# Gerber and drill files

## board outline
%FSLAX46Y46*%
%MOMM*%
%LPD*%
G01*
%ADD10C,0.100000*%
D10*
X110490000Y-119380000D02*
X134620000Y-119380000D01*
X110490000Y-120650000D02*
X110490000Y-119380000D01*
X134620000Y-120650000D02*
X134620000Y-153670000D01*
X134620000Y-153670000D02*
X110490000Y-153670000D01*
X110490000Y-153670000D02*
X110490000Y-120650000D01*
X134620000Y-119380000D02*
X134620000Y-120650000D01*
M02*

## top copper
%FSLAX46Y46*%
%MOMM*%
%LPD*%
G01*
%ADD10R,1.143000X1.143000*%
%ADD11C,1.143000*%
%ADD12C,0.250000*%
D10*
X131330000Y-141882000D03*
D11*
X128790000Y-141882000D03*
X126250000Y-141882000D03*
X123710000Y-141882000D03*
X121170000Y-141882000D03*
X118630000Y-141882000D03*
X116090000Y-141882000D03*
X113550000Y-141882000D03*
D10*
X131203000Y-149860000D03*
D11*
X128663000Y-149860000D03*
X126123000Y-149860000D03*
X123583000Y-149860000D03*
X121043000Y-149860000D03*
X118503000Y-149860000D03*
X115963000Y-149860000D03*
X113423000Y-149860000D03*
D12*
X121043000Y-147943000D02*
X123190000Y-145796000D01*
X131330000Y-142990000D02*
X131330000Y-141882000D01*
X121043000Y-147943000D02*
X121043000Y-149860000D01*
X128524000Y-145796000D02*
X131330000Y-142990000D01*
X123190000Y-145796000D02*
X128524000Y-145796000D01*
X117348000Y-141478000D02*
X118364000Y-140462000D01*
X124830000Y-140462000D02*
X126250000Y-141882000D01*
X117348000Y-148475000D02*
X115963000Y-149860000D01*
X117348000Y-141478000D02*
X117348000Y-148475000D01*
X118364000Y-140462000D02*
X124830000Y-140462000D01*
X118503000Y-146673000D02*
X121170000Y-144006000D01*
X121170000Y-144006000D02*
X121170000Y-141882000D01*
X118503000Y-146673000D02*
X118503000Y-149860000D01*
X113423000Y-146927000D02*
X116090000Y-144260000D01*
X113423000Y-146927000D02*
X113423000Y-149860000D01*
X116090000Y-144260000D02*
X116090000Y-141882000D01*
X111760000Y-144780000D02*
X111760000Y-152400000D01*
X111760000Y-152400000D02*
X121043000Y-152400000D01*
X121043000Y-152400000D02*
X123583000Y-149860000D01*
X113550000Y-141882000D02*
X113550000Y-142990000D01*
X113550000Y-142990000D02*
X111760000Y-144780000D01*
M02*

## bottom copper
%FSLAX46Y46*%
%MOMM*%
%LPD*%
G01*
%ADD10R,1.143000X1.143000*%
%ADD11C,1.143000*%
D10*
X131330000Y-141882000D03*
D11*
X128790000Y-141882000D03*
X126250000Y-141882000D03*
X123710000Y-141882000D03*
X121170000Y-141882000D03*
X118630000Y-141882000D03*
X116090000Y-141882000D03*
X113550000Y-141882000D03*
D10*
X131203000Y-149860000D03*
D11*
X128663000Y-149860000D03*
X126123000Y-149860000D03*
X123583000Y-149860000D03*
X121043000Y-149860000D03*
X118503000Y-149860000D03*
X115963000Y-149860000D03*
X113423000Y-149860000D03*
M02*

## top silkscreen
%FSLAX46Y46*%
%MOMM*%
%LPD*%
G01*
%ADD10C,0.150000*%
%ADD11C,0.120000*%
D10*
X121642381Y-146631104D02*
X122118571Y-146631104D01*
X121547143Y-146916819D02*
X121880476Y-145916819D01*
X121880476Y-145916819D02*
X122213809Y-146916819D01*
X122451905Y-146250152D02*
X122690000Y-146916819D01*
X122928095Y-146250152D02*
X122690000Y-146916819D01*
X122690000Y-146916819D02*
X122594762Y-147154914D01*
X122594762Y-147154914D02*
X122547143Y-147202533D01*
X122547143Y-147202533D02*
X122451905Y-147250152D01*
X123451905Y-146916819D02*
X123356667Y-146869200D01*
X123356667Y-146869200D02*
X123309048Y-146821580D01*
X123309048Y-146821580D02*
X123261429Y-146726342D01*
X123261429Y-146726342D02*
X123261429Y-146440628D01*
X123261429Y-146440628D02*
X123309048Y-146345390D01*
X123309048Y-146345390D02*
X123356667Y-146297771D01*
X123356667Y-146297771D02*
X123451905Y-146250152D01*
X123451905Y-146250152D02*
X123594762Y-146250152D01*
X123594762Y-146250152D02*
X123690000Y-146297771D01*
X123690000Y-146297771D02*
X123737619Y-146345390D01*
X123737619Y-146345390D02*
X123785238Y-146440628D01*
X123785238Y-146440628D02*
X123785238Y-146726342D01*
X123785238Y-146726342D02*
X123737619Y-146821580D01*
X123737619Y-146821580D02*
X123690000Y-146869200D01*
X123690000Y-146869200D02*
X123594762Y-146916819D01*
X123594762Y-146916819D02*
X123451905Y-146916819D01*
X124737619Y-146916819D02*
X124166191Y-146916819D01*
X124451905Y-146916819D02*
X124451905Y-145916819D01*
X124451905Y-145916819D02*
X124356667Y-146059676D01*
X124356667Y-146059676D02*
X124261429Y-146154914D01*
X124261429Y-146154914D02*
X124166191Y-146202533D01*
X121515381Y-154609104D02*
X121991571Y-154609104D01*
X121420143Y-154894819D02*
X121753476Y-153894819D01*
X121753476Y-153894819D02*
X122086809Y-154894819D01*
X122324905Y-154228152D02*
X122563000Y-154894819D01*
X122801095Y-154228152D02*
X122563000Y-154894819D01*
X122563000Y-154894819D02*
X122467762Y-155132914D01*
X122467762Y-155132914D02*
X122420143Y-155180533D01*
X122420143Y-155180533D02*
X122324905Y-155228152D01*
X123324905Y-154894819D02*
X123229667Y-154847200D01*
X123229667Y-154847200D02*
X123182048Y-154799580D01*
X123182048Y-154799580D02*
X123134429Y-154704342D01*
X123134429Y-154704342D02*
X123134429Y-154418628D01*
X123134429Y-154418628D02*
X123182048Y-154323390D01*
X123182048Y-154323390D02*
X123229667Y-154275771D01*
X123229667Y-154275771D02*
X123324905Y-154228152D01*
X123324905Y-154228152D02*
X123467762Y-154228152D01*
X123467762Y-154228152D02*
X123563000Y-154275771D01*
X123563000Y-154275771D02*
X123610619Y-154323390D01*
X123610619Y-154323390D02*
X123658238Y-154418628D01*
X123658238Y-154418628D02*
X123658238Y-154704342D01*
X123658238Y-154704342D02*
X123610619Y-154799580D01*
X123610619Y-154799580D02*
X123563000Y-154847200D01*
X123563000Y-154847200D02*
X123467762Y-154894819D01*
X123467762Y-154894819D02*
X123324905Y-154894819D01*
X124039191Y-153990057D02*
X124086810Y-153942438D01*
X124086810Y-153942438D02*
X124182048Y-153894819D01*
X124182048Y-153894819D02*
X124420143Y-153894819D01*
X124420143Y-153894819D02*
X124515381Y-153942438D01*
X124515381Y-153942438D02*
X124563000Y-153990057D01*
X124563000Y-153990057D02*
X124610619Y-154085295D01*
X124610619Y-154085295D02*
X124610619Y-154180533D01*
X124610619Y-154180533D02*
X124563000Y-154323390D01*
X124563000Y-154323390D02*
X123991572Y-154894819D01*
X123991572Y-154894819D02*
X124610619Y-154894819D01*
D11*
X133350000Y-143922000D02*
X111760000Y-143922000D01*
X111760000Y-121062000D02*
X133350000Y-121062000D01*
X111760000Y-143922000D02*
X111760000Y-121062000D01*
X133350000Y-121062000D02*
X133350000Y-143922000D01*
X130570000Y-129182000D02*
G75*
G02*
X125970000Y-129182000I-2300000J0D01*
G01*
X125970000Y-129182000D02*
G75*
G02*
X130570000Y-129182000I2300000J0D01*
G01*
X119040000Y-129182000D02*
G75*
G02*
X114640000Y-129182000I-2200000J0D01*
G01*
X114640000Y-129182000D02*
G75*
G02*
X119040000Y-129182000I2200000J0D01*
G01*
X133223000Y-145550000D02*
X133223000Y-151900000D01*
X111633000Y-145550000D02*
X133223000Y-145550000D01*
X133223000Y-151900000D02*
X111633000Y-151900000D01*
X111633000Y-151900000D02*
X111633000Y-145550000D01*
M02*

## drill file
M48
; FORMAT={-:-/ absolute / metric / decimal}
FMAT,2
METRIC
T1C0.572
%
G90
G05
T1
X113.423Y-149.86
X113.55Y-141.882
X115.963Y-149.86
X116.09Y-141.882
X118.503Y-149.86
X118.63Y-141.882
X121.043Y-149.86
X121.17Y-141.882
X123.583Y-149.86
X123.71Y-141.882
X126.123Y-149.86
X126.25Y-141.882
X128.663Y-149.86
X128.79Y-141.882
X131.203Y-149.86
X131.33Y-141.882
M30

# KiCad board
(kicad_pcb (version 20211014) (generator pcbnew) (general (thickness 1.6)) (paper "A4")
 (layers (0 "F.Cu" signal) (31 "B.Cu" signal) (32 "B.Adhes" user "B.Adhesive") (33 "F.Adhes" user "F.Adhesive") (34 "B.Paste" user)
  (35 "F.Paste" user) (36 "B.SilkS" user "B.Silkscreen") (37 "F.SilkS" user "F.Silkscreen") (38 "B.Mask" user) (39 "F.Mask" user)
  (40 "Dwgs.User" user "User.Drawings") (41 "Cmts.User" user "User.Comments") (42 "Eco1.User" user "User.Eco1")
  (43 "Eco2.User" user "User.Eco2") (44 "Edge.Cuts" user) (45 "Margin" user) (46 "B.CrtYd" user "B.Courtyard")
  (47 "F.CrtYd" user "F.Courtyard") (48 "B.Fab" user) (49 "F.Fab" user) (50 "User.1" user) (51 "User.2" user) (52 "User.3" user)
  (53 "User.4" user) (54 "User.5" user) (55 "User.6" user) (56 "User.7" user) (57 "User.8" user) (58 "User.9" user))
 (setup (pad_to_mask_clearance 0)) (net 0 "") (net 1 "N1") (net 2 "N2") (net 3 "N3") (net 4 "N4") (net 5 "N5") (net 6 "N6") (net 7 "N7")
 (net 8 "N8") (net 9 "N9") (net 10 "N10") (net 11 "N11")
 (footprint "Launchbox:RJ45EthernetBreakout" (layer "F.Cu") (at 123.19 132.492)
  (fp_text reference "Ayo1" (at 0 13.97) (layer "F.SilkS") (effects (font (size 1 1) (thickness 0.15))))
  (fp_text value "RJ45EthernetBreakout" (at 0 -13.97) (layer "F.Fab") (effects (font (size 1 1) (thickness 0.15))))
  (fp_line (start 10.16 11.43) (end -11.43 11.43) (layer "F.SilkS") (width 0.12))
  (fp_line (start -11.43 -11.43) (end 10.16 -11.43) (layer "F.SilkS") (width 0.12))
  (fp_line (start -11.43 11.43) (end -11.43 -11.43) (layer "F.SilkS") (width 0.12))
  (fp_line (start 10.16 -11.43) (end 10.16 11.43) (layer "F.SilkS") (width 0.12))
  (fp_circle (center 5.08 -3.31) (end 7.38 -3.31) (layer "F.SilkS") (width 0.12) (fill none))
  (fp_circle (center -6.35 -3.31) (end -4.15 -3.31) (layer "F.SilkS") (width 0.12) (fill none))
  (pad "1" thru_hole rect (at 8.14 9.39) (size 1.143 1.143) (drill 0.5715) (layers *.Cu *.Mask) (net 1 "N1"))
  (pad "2" thru_hole circle (at 5.6 9.39) (size 1.143 1.143) (drill 0.5715) (layers *.Cu *.Mask) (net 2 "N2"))
  (pad "3" thru_hole circle (at 3.06 9.39) (size 1.143 1.143) (drill 0.5715) (layers *.Cu *.Mask) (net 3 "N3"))
  (pad "4" thru_hole circle (at 0.52 9.39) (size 1.143 1.143) (drill 0.5715) (layers *.Cu *.Mask) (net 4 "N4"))
  (pad "5" thru_hole circle (at -2.02 9.39) (size 1.143 1.143) (drill 0.5715) (layers *.Cu *.Mask) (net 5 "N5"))
  (pad "6" thru_hole circle (at -4.56 9.39) (size 1.143 1.143) (drill 0.5715) (layers *.Cu *.Mask) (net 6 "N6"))
  (pad "7" thru_hole circle (at -7.1 9.39) (size 1.143 1.143) (drill 0.5715) (layers *.Cu *.Mask) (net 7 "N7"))
  (pad "8" thru_hole circle (at -9.64 9.39) (size 1.143 1.143) (drill 0.5715) (layers *.Cu *.Mask) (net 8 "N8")))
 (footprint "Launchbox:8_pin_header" (layer "F.Cu") (at 123.063 149.86)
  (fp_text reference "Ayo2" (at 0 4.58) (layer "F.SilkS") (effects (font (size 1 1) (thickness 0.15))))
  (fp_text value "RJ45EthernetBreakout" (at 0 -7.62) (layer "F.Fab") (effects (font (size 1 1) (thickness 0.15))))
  (fp_line (start 10.16 -4.31) (end 10.16 2.04) (layer "F.SilkS") (width 0.12))
  (fp_line (start -11.43 -4.31) (end 10.16 -4.31) (layer "F.SilkS") (width 0.12))
  (fp_line (start 10.16 2.04) (end -11.43 2.04) (layer "F.SilkS") (width 0.12))
  (fp_line (start -11.43 2.04) (end -11.43 -4.31) (layer "F.SilkS") (width 0.12))
  (pad "1" thru_hole rect (at 8.14 0) (size 1.143 1.143) (drill 0.5715) (layers *.Cu *.Mask) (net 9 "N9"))
  (pad "2" thru_hole circle (at 5.6 0) (size 1.143 1.143) (drill 0.5715) (layers *.Cu *.Mask) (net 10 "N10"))
  (pad "3" thru_hole circle (at 3.06 0) (size 1.143 1.143) (drill 0.5715) (layers *.Cu *.Mask) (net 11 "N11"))
  (pad "4" thru_hole circle (at 0.52 0) (size 1.143 1.143) (drill 0.5715) (layers *.Cu *.Mask) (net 8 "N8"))
  (pad "5" thru_hole circle (at -2.02 0) (size 1.143 1.143) (drill 0.5715) (layers *.Cu *.Mask) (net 1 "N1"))
  (pad "6" thru_hole circle (at -4.56 0) (size 1.143 1.143) (drill 0.5715) (layers *.Cu *.Mask) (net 5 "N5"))
  (pad "7" thru_hole circle (at -7.1 0) (size 1.143 1.143) (drill 0.5715) (layers *.Cu *.Mask) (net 3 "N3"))
  (pad "8" thru_hole circle (at -9.64 0) (size 1.143 1.143) (drill 0.5715) (layers *.Cu *.Mask) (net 7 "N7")))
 (gr_line (start 110.49 119.38) (end 134.62 119.38) (layer "Edge.Cuts") (width 0.1))
 (gr_line (start 110.49 120.65) (end 110.49 119.38) (layer "Edge.Cuts") (width 0.1))
 (gr_line (start 134.62 120.65) (end 134.62 153.67) (layer "Edge.Cuts") (width 0.1))
 (gr_line (start 134.62 153.67) (end 110.49 153.67) (layer "Edge.Cuts") (width 0.1))
 (gr_line (start 110.49 153.67) (end 110.49 120.65) (layer "Edge.Cuts") (width 0.1))
 (gr_line (start 134.62 119.38) (end 134.62 120.65) (layer "Edge.Cuts") (width 0.1))
 (segment (start 121.043 147.943) (end 123.19 145.796) (width 0.25) (layer "F.Cu") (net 1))
 (segment (start 131.33 142.99) (end 131.33 141.882) (width 0.25) (layer "F.Cu") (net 1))
 (segment (start 121.043 147.943) (end 121.043 149.86) (width 0.25) (layer "F.Cu") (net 1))
 (segment (start 128.524 145.796) (end 131.33 142.99) (width 0.25) (layer "F.Cu") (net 1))
 (segment (start 123.19 145.796) (end 128.524 145.796) (width 0.25) (layer "F.Cu") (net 1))
 (segment (start 117.348 141.478) (end 118.364 140.462) (width 0.25) (layer "F.Cu") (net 3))
 (segment (start 124.83 140.462) (end 126.25 141.882) (width 0.25) (layer "F.Cu") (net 3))
 (segment (start 117.348 148.475) (end 115.963 149.86) (width 0.25) (layer "F.Cu") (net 3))
 (segment (start 117.348 141.478) (end 117.348 148.475) (width 0.25) (layer "F.Cu") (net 3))
 (segment (start 118.364 140.462) (end 124.83 140.462) (width 0.25) (layer "F.Cu") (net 3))
 (segment (start 118.503 146.673) (end 121.17 144.006) (width 0.25) (layer "F.Cu") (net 5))
 (segment (start 121.17 144.006) (end 121.17 141.882) (width 0.25) (layer "F.Cu") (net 5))
 (segment (start 118.503 146.673) (end 118.503 149.86) (width 0.25) (layer "F.Cu") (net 5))
 (segment (start 113.423 146.927) (end 116.09 144.26) (width 0.25) (layer "F.Cu") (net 7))
 (segment (start 113.423 146.927) (end 113.423 149.86) (width 0.25) (layer "F.Cu") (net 7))
 (segment (start 116.09 144.26) (end 116.09 141.882) (width 0.25) (layer "F.Cu") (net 7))
 (segment (start 111.76 144.78) (end 111.76 152.4) (width 0.25) (layer "F.Cu") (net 8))
 (segment (start 111.76 152.4) (end 121.043 152.4) (width 0.25) (layer "F.Cu") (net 8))
 (segment (start 121.043 152.4) (end 123.583 149.86) (width 0.25) (layer "F.Cu") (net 8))
 (segment (start 113.55 141.882) (end 113.55 142.99) (width 0.25) (layer "F.Cu") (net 8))
 (segment (start 113.55 142.99) (end 111.76 144.78) (width 0.25) (layer "F.Cu") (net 8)))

